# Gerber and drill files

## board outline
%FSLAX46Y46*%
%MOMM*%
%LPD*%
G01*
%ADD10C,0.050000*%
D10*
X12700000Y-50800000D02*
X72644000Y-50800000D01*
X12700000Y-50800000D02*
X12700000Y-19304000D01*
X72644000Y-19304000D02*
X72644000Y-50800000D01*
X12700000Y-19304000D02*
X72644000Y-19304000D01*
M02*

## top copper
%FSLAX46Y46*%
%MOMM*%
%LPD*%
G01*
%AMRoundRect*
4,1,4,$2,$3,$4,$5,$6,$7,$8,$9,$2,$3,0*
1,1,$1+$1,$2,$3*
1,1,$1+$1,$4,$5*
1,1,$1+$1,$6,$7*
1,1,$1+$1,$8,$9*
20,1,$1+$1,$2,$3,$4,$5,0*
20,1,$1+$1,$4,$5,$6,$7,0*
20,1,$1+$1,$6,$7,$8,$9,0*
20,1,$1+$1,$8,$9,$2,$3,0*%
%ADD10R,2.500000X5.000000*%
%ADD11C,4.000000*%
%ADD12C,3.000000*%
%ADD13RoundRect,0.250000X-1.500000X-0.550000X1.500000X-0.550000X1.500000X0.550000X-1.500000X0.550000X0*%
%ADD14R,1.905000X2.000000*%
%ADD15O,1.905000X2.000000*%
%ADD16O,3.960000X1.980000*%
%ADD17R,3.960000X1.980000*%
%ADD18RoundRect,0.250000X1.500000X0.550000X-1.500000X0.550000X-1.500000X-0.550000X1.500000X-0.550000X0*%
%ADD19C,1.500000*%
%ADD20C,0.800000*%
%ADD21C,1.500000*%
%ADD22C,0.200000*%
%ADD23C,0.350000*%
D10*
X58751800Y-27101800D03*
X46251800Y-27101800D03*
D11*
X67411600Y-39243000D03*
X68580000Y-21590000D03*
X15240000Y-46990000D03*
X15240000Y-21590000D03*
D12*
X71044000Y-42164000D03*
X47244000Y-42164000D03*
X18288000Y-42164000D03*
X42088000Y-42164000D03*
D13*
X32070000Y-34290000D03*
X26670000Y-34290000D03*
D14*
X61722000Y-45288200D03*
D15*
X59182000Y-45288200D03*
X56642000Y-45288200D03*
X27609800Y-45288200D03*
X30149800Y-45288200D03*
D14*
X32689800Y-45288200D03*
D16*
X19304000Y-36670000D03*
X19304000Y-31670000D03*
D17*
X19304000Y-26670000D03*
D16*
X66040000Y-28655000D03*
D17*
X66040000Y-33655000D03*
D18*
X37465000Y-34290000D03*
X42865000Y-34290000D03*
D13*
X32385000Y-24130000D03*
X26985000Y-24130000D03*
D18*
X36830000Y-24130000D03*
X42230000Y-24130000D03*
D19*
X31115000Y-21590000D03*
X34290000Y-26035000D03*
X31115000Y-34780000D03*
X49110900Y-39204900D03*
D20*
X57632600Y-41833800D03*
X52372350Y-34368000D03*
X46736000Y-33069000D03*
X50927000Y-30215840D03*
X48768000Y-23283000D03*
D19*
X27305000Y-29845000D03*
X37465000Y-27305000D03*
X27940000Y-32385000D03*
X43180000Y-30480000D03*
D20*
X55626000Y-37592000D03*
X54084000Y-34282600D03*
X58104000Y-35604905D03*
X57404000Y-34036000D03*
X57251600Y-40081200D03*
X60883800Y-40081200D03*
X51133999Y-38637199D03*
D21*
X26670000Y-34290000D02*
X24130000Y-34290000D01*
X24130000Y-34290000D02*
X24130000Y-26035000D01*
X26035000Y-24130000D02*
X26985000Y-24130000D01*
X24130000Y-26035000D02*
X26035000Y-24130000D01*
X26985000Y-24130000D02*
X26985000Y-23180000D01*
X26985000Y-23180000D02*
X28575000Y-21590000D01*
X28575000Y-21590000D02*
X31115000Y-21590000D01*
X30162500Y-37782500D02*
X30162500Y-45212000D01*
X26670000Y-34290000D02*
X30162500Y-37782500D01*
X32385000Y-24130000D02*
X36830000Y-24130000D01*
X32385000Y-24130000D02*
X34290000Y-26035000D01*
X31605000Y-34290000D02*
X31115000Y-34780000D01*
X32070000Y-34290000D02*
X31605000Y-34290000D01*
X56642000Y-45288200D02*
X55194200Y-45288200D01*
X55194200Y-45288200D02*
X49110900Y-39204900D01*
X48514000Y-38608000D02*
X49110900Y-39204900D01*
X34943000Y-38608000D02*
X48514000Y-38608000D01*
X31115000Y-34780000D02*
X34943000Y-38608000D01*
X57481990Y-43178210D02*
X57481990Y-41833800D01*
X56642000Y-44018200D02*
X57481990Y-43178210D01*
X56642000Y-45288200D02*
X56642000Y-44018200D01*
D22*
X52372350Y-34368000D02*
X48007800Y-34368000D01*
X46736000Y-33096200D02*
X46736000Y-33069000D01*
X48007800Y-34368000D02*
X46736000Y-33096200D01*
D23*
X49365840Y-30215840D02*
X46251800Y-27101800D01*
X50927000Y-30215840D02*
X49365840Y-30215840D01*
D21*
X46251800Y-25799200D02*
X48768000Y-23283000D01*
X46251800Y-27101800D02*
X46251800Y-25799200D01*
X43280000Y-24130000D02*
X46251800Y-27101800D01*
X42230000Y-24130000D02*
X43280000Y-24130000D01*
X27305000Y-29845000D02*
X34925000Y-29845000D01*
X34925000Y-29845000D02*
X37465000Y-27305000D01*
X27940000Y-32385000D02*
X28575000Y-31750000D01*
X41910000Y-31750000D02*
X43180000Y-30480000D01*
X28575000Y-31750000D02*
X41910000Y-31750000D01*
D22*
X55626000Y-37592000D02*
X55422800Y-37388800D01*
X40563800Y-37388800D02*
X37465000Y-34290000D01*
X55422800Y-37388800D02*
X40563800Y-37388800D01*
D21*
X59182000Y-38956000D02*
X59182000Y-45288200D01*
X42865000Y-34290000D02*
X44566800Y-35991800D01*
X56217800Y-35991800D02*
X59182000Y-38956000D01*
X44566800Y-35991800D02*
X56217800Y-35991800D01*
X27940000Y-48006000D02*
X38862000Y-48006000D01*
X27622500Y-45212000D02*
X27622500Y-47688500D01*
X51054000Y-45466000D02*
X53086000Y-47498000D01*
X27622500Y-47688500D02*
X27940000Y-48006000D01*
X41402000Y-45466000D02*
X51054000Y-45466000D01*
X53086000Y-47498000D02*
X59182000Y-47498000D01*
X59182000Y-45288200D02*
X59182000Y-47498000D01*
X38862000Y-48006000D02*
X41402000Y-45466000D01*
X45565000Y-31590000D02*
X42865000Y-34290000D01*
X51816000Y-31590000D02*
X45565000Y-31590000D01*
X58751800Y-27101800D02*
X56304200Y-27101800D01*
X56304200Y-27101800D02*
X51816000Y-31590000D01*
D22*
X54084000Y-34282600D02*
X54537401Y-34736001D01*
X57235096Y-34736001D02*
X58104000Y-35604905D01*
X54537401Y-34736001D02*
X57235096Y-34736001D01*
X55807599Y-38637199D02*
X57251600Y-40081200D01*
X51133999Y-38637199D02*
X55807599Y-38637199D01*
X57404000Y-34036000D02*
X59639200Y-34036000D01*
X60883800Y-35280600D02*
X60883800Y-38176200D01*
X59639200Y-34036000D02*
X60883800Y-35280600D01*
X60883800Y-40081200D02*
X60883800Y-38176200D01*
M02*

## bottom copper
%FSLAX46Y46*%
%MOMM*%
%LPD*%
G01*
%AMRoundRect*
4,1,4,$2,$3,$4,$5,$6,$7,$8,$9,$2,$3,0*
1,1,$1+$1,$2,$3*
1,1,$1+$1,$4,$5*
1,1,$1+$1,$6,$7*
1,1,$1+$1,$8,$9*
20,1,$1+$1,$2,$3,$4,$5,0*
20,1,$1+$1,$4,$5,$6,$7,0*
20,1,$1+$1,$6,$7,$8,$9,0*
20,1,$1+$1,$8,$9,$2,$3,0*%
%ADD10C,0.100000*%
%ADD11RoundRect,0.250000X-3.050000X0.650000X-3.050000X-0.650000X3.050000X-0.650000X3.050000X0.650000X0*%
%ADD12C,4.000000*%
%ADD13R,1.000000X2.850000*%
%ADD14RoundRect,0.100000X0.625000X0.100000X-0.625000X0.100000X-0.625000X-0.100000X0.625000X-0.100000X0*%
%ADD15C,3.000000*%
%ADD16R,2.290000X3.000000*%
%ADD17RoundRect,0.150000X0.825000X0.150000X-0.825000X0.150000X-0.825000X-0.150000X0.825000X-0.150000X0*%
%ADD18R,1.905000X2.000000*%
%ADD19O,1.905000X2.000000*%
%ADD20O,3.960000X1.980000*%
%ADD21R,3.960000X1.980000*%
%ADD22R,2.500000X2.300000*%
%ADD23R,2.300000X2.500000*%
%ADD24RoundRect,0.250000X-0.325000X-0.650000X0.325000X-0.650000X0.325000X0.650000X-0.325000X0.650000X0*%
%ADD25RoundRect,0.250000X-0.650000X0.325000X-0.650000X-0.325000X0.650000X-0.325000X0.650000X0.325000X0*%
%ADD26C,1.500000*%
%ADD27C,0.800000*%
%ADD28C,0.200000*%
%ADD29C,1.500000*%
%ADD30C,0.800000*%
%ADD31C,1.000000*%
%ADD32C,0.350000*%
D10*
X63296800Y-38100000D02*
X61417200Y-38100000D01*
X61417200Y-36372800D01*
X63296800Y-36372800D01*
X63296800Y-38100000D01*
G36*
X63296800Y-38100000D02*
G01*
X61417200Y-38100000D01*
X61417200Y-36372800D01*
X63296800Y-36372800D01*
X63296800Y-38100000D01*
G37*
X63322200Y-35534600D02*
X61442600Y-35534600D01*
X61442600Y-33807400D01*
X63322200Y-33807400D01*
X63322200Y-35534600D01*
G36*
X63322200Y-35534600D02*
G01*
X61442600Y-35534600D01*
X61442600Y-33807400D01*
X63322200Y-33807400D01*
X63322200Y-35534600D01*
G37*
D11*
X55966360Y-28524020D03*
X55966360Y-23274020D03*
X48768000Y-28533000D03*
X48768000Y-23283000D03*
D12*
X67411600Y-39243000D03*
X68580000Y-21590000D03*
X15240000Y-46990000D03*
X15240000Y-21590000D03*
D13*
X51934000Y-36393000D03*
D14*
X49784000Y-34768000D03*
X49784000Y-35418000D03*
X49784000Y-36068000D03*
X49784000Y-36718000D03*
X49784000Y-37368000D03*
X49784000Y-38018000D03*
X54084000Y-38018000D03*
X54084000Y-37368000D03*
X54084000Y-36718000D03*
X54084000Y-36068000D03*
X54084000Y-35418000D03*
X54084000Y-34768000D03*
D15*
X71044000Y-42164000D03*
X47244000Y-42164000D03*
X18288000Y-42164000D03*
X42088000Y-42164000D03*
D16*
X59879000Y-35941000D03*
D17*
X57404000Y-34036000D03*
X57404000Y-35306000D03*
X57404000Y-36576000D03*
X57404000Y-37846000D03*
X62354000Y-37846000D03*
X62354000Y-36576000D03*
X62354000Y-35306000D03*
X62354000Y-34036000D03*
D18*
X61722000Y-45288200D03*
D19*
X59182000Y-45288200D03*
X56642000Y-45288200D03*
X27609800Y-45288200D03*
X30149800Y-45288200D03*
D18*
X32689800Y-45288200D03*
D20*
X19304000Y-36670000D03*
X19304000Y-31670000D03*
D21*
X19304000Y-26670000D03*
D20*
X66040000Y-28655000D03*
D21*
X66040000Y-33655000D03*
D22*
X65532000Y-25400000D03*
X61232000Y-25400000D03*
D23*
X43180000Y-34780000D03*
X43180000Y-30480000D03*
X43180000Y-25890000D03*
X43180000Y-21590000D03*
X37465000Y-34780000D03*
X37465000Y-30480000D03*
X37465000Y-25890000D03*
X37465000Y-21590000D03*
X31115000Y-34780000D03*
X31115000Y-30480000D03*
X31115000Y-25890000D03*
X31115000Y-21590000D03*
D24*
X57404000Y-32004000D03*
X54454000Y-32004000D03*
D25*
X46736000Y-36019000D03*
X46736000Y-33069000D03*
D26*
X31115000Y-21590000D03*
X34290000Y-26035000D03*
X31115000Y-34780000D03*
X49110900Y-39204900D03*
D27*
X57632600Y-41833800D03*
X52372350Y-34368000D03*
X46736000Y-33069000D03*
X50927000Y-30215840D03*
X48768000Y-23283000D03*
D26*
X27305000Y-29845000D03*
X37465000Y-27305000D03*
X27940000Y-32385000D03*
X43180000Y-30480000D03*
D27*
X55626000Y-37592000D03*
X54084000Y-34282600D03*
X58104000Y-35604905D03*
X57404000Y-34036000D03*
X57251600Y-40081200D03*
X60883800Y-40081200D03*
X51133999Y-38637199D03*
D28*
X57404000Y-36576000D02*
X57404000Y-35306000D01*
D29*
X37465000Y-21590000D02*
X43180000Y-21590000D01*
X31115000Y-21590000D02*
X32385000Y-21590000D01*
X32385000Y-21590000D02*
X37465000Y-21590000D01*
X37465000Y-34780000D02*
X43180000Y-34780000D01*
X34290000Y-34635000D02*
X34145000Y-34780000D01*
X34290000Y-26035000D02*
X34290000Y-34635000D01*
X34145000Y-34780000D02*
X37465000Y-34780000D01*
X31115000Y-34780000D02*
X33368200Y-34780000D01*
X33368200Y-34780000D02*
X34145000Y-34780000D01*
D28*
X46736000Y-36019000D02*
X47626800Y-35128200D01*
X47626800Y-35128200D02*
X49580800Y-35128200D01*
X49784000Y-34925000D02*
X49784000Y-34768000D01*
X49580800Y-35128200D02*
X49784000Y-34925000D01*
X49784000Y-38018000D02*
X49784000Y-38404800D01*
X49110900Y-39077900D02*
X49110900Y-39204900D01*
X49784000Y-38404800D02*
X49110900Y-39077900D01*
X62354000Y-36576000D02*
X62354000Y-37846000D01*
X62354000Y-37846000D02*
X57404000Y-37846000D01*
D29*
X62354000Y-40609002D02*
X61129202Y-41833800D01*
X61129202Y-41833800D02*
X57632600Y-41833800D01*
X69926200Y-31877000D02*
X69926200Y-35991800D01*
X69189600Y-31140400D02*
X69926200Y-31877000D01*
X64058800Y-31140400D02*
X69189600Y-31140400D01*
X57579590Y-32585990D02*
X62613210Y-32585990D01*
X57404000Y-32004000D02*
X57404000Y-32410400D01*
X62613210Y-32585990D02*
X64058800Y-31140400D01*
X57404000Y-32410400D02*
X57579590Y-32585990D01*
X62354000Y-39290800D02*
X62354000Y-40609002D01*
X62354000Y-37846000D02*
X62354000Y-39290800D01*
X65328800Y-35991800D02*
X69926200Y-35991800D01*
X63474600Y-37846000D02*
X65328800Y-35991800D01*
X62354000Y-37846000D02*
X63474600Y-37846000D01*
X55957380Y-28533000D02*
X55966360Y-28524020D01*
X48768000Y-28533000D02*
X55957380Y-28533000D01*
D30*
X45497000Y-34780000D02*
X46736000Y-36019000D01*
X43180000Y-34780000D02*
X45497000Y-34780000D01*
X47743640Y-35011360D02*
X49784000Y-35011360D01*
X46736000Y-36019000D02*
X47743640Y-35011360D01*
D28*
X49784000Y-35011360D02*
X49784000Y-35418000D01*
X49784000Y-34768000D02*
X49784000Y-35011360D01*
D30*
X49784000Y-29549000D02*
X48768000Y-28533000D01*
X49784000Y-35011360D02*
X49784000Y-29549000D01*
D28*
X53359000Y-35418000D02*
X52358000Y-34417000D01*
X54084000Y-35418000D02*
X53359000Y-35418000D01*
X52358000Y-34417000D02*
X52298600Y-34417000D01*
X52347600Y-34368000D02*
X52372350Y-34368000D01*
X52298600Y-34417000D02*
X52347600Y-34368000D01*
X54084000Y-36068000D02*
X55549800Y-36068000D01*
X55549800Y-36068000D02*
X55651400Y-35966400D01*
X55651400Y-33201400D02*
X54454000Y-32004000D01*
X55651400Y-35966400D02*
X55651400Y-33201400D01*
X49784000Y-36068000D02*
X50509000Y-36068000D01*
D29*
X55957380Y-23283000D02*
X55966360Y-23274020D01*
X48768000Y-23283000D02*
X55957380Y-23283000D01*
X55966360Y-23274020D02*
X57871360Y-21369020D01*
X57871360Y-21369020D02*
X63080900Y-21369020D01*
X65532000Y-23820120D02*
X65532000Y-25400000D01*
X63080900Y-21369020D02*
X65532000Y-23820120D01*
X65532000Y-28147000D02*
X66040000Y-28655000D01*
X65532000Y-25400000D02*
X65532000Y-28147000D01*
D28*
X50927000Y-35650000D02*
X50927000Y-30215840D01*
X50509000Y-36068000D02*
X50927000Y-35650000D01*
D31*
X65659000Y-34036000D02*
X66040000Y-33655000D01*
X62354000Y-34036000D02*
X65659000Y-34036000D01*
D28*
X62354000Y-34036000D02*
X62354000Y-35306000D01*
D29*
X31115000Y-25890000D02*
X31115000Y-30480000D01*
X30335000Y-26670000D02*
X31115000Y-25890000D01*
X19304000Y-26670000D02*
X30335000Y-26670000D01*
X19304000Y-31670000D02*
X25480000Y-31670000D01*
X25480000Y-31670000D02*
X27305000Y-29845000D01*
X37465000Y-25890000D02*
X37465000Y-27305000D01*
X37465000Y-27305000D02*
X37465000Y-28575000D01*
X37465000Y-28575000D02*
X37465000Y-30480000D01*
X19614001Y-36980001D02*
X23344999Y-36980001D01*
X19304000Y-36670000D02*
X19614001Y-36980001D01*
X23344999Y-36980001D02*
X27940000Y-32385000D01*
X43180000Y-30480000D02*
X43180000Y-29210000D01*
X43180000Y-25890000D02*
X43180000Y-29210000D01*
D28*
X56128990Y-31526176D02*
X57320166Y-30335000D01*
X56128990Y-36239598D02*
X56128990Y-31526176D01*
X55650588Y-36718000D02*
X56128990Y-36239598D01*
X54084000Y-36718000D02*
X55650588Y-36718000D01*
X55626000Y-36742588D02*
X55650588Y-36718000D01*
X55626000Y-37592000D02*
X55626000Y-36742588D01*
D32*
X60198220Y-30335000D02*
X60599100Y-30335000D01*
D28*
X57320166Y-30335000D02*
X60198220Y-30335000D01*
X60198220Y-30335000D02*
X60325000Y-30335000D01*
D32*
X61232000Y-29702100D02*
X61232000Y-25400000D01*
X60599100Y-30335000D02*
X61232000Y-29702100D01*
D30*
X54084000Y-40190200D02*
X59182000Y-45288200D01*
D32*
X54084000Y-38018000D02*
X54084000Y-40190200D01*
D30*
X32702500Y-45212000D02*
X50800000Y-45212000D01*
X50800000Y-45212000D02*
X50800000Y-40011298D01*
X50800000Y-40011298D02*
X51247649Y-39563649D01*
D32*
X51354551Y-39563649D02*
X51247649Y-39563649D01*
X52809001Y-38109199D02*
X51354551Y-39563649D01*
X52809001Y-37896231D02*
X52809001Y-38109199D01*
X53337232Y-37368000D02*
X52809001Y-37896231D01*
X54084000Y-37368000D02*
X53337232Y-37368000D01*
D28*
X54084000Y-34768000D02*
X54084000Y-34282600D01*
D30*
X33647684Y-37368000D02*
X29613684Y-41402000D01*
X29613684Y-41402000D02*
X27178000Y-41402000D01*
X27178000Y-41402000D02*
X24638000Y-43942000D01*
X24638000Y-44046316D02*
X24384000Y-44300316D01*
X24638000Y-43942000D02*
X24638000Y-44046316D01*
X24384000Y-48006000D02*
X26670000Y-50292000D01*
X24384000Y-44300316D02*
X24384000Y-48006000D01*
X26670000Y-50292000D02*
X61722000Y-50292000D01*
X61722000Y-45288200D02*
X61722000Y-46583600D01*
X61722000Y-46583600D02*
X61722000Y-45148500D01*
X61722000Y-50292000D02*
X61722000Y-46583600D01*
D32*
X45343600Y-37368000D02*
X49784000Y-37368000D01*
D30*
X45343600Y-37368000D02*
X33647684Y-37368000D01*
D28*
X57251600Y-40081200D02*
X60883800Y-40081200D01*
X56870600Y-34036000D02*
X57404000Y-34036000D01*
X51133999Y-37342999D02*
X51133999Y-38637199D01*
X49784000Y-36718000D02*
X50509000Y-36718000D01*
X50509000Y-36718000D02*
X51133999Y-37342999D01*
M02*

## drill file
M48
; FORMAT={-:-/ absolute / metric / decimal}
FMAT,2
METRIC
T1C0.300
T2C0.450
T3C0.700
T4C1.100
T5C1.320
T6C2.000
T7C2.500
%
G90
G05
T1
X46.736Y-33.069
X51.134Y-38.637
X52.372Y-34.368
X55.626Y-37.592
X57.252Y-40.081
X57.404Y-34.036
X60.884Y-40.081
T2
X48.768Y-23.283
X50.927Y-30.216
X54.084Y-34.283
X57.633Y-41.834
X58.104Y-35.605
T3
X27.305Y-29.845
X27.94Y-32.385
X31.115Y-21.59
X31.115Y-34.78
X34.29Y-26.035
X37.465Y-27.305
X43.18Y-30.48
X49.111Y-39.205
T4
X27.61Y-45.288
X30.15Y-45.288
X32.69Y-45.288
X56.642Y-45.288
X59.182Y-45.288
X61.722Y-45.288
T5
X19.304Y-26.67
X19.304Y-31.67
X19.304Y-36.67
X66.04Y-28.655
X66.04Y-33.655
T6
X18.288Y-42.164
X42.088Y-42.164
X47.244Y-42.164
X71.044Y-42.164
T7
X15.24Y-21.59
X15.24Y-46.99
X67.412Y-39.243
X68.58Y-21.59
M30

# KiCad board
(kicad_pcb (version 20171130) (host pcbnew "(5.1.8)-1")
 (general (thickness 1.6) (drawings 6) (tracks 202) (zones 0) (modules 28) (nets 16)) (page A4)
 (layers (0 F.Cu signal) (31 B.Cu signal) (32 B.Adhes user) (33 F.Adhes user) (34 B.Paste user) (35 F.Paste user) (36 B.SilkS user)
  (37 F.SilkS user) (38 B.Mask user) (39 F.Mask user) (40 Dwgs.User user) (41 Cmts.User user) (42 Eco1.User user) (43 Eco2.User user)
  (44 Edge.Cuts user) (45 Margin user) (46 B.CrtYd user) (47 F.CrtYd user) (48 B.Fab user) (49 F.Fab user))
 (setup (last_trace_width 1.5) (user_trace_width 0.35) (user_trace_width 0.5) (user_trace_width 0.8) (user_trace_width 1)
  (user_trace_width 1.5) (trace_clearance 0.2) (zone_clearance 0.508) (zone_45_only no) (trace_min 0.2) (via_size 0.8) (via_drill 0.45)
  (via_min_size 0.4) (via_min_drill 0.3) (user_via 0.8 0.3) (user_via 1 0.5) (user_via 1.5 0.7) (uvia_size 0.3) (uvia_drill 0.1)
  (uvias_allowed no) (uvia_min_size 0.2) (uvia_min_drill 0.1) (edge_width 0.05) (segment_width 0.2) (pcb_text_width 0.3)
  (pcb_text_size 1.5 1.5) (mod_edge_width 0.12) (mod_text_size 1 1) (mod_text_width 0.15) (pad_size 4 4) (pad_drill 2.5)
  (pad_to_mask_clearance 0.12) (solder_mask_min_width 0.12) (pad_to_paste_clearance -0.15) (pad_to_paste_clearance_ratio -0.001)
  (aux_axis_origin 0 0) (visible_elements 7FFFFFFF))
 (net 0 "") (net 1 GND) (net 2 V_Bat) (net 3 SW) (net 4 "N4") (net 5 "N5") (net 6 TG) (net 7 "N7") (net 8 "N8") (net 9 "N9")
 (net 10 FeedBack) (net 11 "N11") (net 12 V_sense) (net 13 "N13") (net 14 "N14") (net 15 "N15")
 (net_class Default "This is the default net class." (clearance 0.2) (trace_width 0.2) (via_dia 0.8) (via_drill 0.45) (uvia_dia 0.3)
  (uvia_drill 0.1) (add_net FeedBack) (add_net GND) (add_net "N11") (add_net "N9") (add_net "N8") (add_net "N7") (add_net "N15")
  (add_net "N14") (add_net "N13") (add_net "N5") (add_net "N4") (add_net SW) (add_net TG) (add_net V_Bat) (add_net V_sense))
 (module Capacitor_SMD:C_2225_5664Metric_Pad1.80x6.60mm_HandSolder (layer B.Cu) (at 55.96636 25.89902 270)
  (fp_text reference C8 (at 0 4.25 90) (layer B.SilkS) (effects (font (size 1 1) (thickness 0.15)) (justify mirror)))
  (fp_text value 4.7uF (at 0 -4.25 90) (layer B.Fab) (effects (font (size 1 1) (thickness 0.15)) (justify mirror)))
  (pad 2 smd roundrect (at 2.625 0 270) (size 1.8 6.6) (layers B.Cu B.Paste B.Mask) (roundrect_rratio 0.138889) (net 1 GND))
  (pad 1 smd roundrect (at -2.625 0 270) (size 1.8 6.6) (layers B.Cu B.Paste B.Mask) (roundrect_rratio 0.138889) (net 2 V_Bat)))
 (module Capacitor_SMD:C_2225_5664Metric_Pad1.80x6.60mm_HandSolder (layer B.Cu) (at 48.768 25.908 270)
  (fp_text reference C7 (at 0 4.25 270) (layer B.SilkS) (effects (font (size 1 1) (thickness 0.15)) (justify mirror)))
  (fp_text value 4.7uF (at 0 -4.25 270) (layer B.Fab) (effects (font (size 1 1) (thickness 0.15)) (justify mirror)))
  (pad 2 smd roundrect (at 2.625 0 270) (size 1.8 6.6) (layers B.Cu B.Paste B.Mask) (roundrect_rratio 0.138889) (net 1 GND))
  (pad 1 smd roundrect (at -2.625 0 270) (size 1.8 6.6) (layers B.Cu B.Paste B.Mask) (roundrect_rratio 0.138889) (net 2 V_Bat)))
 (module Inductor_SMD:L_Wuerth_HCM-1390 (layer F.Cu) (at 52.5018 27.1018)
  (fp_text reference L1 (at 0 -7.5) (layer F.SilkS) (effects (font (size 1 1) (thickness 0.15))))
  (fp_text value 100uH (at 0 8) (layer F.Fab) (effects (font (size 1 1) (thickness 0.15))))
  (pad 2 smd rect (at 6.25 0) (size 2.5 5) (layers F.Cu F.Paste F.Mask) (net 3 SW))
  (pad 1 smd rect (at -6.25 0) (size 2.5 5) (layers F.Cu F.Paste F.Mask) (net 2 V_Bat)))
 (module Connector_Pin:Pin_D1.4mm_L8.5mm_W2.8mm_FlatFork (layer F.Cu) (at 67.4116 39.243)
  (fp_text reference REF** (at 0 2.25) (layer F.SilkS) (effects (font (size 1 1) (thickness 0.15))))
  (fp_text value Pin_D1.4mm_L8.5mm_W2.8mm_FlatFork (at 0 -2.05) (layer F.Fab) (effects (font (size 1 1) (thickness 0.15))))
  (pad 1 thru_hole circle (at 0 0) (size 4 4) (drill 2.5) (layers *.Cu *.Mask)))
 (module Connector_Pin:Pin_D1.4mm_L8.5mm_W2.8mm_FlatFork (layer F.Cu) (at 68.58 21.59)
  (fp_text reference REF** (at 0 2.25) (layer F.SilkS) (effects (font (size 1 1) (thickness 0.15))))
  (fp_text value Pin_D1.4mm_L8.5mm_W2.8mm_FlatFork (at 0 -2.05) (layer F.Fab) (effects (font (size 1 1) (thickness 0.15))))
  (pad 1 thru_hole circle (at 0 0) (size 4 4) (drill 2.5) (layers *.Cu *.Mask)))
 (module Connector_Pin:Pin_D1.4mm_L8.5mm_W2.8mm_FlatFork (layer F.Cu) (at 15.24 46.99)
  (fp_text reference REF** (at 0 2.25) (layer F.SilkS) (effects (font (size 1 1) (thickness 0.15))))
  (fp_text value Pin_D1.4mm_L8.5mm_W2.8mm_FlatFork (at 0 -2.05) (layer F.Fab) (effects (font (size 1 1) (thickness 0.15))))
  (pad 1 thru_hole circle (at 0 0) (size 4 4) (drill 2.5) (layers *.Cu *.Mask)))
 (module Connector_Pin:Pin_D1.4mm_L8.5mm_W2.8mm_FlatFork (layer F.Cu) (at 15.24 21.59)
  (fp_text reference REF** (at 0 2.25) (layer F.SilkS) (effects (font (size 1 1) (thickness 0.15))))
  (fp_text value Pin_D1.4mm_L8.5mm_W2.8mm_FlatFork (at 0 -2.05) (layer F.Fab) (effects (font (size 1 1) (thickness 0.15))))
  (pad 1 thru_hole circle (at 0 0) (size 4 4) (drill 2.5) (layers *.Cu *.Mask)))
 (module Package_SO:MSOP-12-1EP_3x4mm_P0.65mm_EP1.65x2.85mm (layer B.Cu) (at 51.934 36.393 180)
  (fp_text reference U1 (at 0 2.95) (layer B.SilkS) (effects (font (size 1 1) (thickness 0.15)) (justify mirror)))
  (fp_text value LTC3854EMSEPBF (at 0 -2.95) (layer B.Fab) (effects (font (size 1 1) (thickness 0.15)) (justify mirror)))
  (pad "" smd roundrect (at 0.41 -0.71 180) (size 0.67 1.15) (layers B.Paste) (roundrect_rratio 0.25))
  (pad "" smd roundrect (at 0.41 0.71 180) (size 0.67 1.15) (layers B.Paste) (roundrect_rratio 0.25))
  (pad "" smd roundrect (at -0.41 -0.71 180) (size 0.67 1.15) (layers B.Paste) (roundrect_rratio 0.25))
  (pad "" smd roundrect (at -0.41 0.71 180) (size 0.67 1.15) (layers B.Paste) (roundrect_rratio 0.25))
  (pad 13 smd rect (at 0 0 180) (size 1 2.85) (layers B.Cu B.Mask))
  (pad 12 smd roundrect (at 2.15 1.625 180) (size 1.45 0.4) (layers B.Cu B.Paste B.Mask) (roundrect_rratio 0.25) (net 1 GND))
  (pad 11 smd roundrect (at 2.15 0.975 180) (size 1.45 0.4) (layers B.Cu B.Paste B.Mask) (roundrect_rratio 0.25) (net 1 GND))
  (pad 10 smd roundrect (at 2.15 0.325 180) (size 1.45 0.4) (layers B.Cu B.Paste B.Mask) (roundrect_rratio 0.25) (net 2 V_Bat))
  (pad 9 smd roundrect (at 2.15 -0.325 180) (size 1.45 0.4) (layers B.Cu B.Paste B.Mask) (roundrect_rratio 0.25) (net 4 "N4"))
  (pad 8 smd roundrect (at 2.15 -0.975 180) (size 1.45 0.4) (layers B.Cu B.Paste B.Mask) (roundrect_rratio 0.25) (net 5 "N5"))
  (pad 7 smd roundrect (at 2.15 -1.625 180) (size 1.45 0.4) (layers B.Cu B.Paste B.Mask) (roundrect_rratio 0.25) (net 1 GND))
  (pad 6 smd roundrect (at -2.15 -1.625 180) (size 1.45 0.4) (layers B.Cu B.Paste B.Mask) (roundrect_rratio 0.25) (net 3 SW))
  (pad 5 smd roundrect (at -2.15 -0.975 180) (size 1.45 0.4) (layers B.Cu B.Paste B.Mask) (roundrect_rratio 0.25) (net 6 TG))
  (pad 4 smd roundrect (at -2.15 -0.325 180) (size 1.45 0.4) (layers B.Cu B.Paste B.Mask) (roundrect_rratio 0.25) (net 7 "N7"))
  (pad 3 smd roundrect (at -2.15 0.325 180) (size 1.45 0.4) (layers B.Cu B.Paste B.Mask) (roundrect_rratio 0.25) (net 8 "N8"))
  (pad 2 smd roundrect (at -2.15 0.975 180) (size 1.45 0.4) (layers B.Cu B.Paste B.Mask) (roundrect_rratio 0.25) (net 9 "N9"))
  (pad 1 smd roundrect (at -2.15 1.625 180) (size 1.45 0.4) (layers B.Cu B.Paste B.Mask) (roundrect_rratio 0.25) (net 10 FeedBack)))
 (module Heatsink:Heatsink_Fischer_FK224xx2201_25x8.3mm (layer F.Cu) (at 47.244 42.164)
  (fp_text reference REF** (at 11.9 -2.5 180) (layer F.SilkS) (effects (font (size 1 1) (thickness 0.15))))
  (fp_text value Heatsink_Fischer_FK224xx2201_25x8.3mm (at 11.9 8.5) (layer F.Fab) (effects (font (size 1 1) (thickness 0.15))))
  (pad 1 thru_hole circle (at 23.8 0) (size 3 3) (drill 2) (layers *.Cu *.Mask))
  (pad 1 thru_hole circle (at 0 0) (size 3 3) (drill 2) (layers *.Cu *.Mask)))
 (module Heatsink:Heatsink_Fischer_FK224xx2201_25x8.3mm (layer F.Cu) (at 18.288 42.164)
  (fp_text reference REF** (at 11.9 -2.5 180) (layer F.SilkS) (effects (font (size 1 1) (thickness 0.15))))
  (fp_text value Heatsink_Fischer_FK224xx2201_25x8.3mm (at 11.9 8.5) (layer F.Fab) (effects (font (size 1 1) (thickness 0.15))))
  (pad 1 thru_hole circle (at 0 0) (size 3 3) (drill 2) (layers *.Cu *.Mask))
  (pad 1 thru_hole circle (at 23.8 0) (size 3 3) (drill 2) (layers *.Cu *.Mask)))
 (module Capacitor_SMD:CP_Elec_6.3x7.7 (layer F.Cu) (at 29.37 34.29)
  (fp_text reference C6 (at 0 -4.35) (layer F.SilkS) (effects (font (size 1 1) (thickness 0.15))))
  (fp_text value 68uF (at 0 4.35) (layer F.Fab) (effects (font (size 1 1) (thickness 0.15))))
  (pad 2 smd roundrect (at 2.7 0) (size 3.5 1.6) (layers F.Cu F.Paste F.Mask) (roundrect_rratio 0.15625) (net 1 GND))
  (pad 1 smd roundrect (at -2.7 0) (size 3.5 1.6) (layers F.Cu F.Paste F.Mask) (roundrect_rratio 0.15625) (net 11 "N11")))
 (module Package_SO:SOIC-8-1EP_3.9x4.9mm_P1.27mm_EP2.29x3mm (layer B.Cu) (at 59.879 35.941 180)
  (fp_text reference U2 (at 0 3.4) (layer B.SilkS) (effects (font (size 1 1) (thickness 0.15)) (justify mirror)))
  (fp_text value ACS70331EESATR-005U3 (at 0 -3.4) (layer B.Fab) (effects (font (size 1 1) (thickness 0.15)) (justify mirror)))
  (pad "" smd roundrect (at 0.57 -0.75 180) (size 0.92 1.21) (layers B.Paste) (roundrect_rratio 0.25))
  (pad "" smd roundrect (at 0.57 0.75 180) (size 0.92 1.21) (layers B.Paste) (roundrect_rratio 0.25))
  (pad "" smd roundrect (at -0.57 -0.75 180) (size 0.92 1.21) (layers B.Paste) (roundrect_rratio 0.25))
  (pad "" smd roundrect (at -0.57 0.75 180) (size 0.92 1.21) (layers B.Paste) (roundrect_rratio 0.25))
  (pad 9 smd rect (at 0 0 180) (size 2.29 3) (layers B.Cu B.Mask))
  (pad 8 smd roundrect (at 2.475 1.905 180) (size 1.95 0.6) (layers B.Cu B.Paste B.Mask) (roundrect_rratio 0.25) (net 4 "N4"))
  (pad 7 smd roundrect (at 2.475 0.635 180) (size 1.95 0.6) (layers B.Cu B.Paste B.Mask) (roundrect_rratio 0.25) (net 10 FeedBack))
  (pad 6 smd roundrect (at 2.475 -0.635 180) (size 1.95 0.6) (layers B.Cu B.Paste B.Mask) (roundrect_rratio 0.25))
  (pad 5 smd roundrect (at 2.475 -1.905 180) (size 1.95 0.6) (layers B.Cu B.Paste B.Mask) (roundrect_rratio 0.25) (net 1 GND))
  (pad 4 smd roundrect (at -2.475 -1.905 180) (size 1.95 0.6) (layers B.Cu B.Paste B.Mask) (roundrect_rratio 0.25) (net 1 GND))
  (pad 3 smd roundrect (at -2.475 -0.635 180) (size 1.95 0.6) (layers B.Cu B.Paste B.Mask) (roundrect_rratio 0.25) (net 1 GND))
  (pad 2 smd roundrect (at -2.475 0.635 180) (size 1.95 0.6) (layers B.Cu B.Paste B.Mask) (roundrect_rratio 0.25) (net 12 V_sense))
  (pad 1 smd roundrect (at -2.475 1.905 180) (size 1.95 0.6) (layers B.Cu B.Paste B.Mask) (roundrect_rratio 0.25) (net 12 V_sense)))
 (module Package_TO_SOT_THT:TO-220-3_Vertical (layer F.Cu) (at 61.722 45.2882 180)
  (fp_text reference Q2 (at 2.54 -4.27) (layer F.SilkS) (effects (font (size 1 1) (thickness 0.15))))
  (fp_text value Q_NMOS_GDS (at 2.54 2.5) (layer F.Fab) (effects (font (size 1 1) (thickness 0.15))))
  (pad 1 thru_hole rect (at 0 0 180) (size 1.905 2) (drill 1.1) (layers *.Cu *.Mask) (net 5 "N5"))
  (pad 2 thru_hole oval (at 2.54 0 180) (size 1.905 2) (drill 1.1) (layers *.Cu *.Mask) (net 3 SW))
  (pad 3 thru_hole oval (at 5.08 0 180) (size 1.905 2) (drill 1.1) (layers *.Cu *.Mask) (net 1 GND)))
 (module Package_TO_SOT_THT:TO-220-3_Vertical (layer F.Cu) (at 32.6898 45.2882 180)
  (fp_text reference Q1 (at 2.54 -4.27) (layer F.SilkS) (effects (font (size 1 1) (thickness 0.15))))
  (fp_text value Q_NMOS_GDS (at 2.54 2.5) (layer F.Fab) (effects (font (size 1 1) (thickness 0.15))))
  (pad 3 thru_hole oval (at 5.08 0 180) (size 1.905 2) (drill 1.1) (layers *.Cu *.Mask) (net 3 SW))
  (pad 2 thru_hole oval (at 2.54 0 180) (size 1.905 2) (drill 1.1) (layers *.Cu *.Mask) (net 11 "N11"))
  (pad 1 thru_hole rect (at 0 0 180) (size 1.905 2) (drill 1.1) (layers *.Cu *.Mask) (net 6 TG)))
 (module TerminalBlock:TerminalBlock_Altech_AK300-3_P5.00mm (layer F.Cu) (at 19.304 26.67 270)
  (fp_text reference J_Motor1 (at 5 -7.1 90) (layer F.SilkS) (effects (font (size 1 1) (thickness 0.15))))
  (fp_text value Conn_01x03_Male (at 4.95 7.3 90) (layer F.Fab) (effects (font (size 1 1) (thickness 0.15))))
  (pad 3 thru_hole oval (at 10 0 270) (size 1.98 3.96) (drill 1.32) (layers *.Cu *.Mask) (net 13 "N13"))
  (pad 2 thru_hole oval (at 5 0 270) (size 1.98 3.96) (drill 1.32) (layers *.Cu *.Mask) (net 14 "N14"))
  (pad 1 thru_hole rect (at 0 0 270) (size 1.98 3.96) (drill 1.32) (layers *.Cu *.Mask) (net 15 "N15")))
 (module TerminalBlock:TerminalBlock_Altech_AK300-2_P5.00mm (layer F.Cu) (at 66.04 33.655 90)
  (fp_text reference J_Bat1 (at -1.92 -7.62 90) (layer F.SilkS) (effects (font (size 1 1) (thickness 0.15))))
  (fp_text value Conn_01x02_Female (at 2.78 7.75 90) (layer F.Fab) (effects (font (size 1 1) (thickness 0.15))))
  (pad 2 thru_hole oval (at 5 0 90) (size 1.98 3.96) (drill 1.32) (layers *.Cu *.Mask) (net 2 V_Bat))
  (pad 1 thru_hole rect (at 0 0 90) (size 1.98 3.96) (drill 1.32) (layers *.Cu *.Mask) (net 12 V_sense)))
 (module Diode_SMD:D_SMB (layer B.Cu) (at 63.382 25.4)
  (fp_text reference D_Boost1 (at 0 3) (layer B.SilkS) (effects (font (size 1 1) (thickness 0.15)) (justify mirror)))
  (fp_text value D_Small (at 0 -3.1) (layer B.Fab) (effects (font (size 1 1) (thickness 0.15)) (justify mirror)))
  (pad 2 smd rect (at 2.15 0) (size 2.5 2.3) (layers B.Cu B.Paste B.Mask) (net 2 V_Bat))
  (pad 1 smd rect (at -2.15 0) (size 2.5 2.3) (layers B.Cu B.Paste B.Mask) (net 7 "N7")))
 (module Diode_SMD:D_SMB (layer B.Cu) (at 43.18 32.63 270)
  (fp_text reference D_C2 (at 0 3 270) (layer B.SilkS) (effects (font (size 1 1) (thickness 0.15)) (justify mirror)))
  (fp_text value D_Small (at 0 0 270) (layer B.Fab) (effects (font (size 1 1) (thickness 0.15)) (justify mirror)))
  (pad 2 smd rect (at 2.15 0 270) (size 2.5 2.3) (layers B.Cu B.Paste B.Mask) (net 1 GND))
  (pad 1 smd rect (at -2.15 0 270) (size 2.5 2.3) (layers B.Cu B.Paste B.Mask) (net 13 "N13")))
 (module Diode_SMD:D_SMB (layer B.Cu) (at 43.18 23.74 270)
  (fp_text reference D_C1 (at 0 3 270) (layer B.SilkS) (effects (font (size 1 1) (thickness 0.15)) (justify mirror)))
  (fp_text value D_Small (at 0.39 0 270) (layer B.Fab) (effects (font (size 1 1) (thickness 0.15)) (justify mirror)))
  (pad 2 smd rect (at 2.15 0 270) (size 2.5 2.3) (layers B.Cu B.Paste B.Mask) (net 13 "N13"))
  (pad 1 smd rect (at -2.15 0 270) (size 2.5 2.3) (layers B.Cu B.Paste B.Mask) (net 11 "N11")))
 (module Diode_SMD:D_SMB (layer B.Cu) (at 37.465 32.63 270)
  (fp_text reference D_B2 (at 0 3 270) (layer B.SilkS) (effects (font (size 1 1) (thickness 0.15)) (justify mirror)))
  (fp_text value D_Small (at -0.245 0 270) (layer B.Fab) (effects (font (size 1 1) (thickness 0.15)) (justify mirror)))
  (pad 2 smd rect (at 2.15 0 270) (size 2.5 2.3) (layers B.Cu B.Paste B.Mask) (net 1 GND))
  (pad 1 smd rect (at -2.15 0 270) (size 2.5 2.3) (layers B.Cu B.Paste B.Mask) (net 14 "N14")))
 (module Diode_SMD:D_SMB (layer B.Cu) (at 37.465 23.74 270)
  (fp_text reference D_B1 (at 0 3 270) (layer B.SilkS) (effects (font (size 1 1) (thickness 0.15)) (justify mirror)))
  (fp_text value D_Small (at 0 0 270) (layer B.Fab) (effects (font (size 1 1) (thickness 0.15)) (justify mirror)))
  (pad 2 smd rect (at 2.15 0 270) (size 2.5 2.3) (layers B.Cu B.Paste B.Mask) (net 14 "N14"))
  (pad 1 smd rect (at -2.15 0 270) (size 2.5 2.3) (layers B.Cu B.Paste B.Mask) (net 11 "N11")))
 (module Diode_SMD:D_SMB (layer B.Cu) (at 31.115 32.63 270)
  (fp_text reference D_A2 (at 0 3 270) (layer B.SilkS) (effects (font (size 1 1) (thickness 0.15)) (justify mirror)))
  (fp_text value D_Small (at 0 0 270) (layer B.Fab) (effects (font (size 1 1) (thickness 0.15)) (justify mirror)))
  (pad 2 smd rect (at 2.15 0 270) (size 2.5 2.3) (layers B.Cu B.Paste B.Mask) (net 1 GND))
  (pad 1 smd rect (at -2.15 0 270) (size 2.5 2.3) (layers B.Cu B.Paste B.Mask) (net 15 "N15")))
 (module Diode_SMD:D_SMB (layer B.Cu) (at 31.115 23.74 270)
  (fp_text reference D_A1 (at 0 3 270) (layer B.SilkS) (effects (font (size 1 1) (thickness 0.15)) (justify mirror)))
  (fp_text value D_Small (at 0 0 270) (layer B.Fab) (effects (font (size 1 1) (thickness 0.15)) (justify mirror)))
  (pad 2 smd rect (at 2.15 0 270) (size 2.5 2.3) (layers B.Cu B.Paste B.Mask) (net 15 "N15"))
  (pad 1 smd rect (at -2.15 0 270) (size 2.5 2.3) (layers B.Cu B.Paste B.Mask) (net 11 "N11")))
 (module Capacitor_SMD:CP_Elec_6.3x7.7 (layer F.Cu) (at 40.165 34.29 180)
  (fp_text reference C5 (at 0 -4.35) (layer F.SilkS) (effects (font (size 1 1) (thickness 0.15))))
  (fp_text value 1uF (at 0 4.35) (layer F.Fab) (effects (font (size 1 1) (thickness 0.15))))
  (pad 2 smd roundrect (at 2.7 0 180) (size 3.5 1.6) (layers F.Cu F.Paste F.Mask) (roundrect_rratio 0.15625) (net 7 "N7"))
  (pad 1 smd roundrect (at -2.7 0 180) (size 3.5 1.6) (layers F.Cu F.Paste F.Mask) (roundrect_rratio 0.15625) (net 3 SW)))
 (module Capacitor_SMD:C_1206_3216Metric (layer B.Cu) (at 55.929 32.004)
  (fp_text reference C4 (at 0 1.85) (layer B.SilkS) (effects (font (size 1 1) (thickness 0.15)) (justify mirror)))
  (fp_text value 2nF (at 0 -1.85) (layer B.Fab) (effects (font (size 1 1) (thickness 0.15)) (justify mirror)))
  (pad 2 smd roundrect (at 1.475 0) (size 1.15 1.8) (layers B.Cu B.Paste B.Mask) (roundrect_rratio 0.217391) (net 1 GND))
  (pad 1 smd roundrect (at -1.475 0) (size 1.15 1.8) (layers B.Cu B.Paste B.Mask) (roundrect_rratio 0.217391) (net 8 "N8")))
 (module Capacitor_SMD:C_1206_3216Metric (layer B.Cu) (at 46.736 34.544 270)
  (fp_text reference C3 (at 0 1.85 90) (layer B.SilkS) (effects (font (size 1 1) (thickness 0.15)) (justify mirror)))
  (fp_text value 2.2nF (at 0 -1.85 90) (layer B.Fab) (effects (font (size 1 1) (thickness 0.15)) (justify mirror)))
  (pad 2 smd roundrect (at 1.475 0 270) (size 1.15 1.8) (layers B.Cu B.Paste B.Mask) (roundrect_rratio 0.217391) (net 1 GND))
  (pad 1 smd roundrect (at -1.475 0 270) (size 1.15 1.8) (layers B.Cu B.Paste B.Mask) (roundrect_rratio 0.217391) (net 9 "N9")))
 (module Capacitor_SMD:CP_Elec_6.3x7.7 (layer F.Cu) (at 29.685 24.13)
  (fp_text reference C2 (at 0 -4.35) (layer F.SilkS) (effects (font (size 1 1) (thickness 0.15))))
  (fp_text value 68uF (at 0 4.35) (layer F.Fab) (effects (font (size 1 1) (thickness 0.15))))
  (pad 2 smd roundrect (at 2.7 0) (size 3.5 1.6) (layers F.Cu F.Paste F.Mask) (roundrect_rratio 0.15625) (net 1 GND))
  (pad 1 smd roundrect (at -2.7 0) (size 3.5 1.6) (layers F.Cu F.Paste F.Mask) (roundrect_rratio 0.15625) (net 11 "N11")))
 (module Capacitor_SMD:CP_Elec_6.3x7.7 (layer F.Cu) (at 39.53 24.13 180)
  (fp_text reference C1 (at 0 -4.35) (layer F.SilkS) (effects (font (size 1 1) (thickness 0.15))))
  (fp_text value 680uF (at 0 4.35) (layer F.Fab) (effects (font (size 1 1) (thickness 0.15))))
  (pad 2 smd roundrect (at 2.7 0 180) (size 3.5 1.6) (layers F.Cu F.Paste F.Mask) (roundrect_rratio 0.15625) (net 1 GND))
  (pad 1 smd roundrect (at -2.7 0 180) (size 3.5 1.6) (layers F.Cu F.Paste F.Mask) (roundrect_rratio 0.15625) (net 2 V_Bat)))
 (gr_poly (pts (xy 63.2968 38.1) (xy 61.4172 38.1) (xy 61.4172 36.3728) (xy 63.2968 36.3728)) (layer B.Cu) (width 0.1))
 (gr_poly (pts (xy 63.3222 35.5346) (xy 61.4426 35.5346) (xy 61.4426 33.8074) (xy 63.3222 33.8074)) (layer B.Cu) (width 0.1))
 (gr_line (start 12.7 50.8) (end 72.644 50.8) (layer Edge.Cuts) (width 0.05))
 (gr_line (start 12.7 50.8) (end 12.7 19.304) (layer Edge.Cuts) (width 0.05))
 (gr_line (start 72.644 19.304) (end 72.644 50.8) (layer Edge.Cuts) (width 0.05))
 (gr_line (start 12.7 19.304) (end 72.644 19.304) (layer Edge.Cuts) (width 0.05))
 (segment (start 57.404 36.576) (end 57.404 35.306) (width 0.2) (layer B.Cu) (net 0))
 (segment (start 37.465 21.59) (end 43.18 21.59) (width 1.5) (layer B.Cu) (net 11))
 (segment (start 26.67 34.29) (end 24.13 34.29) (width 1.5) (layer F.Cu) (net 11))
 (segment (start 24.13 34.29) (end 24.13 26.035) (width 1.5) (layer F.Cu) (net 11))
 (segment (start 26.035 24.13) (end 26.985 24.13) (width 1.5) (layer F.Cu) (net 11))
 (segment (start 24.13 26.035) (end 26.035 24.13) (width 1.5) (layer F.Cu) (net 11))
 (segment (start 26.985 24.13) (end 26.985 23.18) (width 1.5) (layer F.Cu) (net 11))
 (segment (start 26.985 23.18) (end 28.575 21.59) (width 1.5) (layer F.Cu) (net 11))
 (via (at 31.115 21.59) (size 1.5) (drill 0.7) (layers F.Cu B.Cu) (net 11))
 (segment (start 28.575 21.59) (end 31.115 21.59) (width 1.5) (layer F.Cu) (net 11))
 (segment (start 31.115 21.59) (end 32.385 21.59) (width 1.5) (layer B.Cu) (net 11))
 (segment (start 32.385 21.59) (end 37.465 21.59) (width 1.5) (layer B.Cu) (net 11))
 (segment (start 30.1625 37.7825) (end 30.1625 45.212) (width 1.5) (layer F.Cu) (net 11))
 (segment (start 26.67 34.29) (end 30.1625 37.7825) (width 1.5) (layer F.Cu) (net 11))
 (segment (start 37.465 34.78) (end 43.18 34.78) (width 1.5) (layer B.Cu) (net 1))
 (segment (start 32.385 24.13) (end 36.83 24.13) (width 1.5) (layer F.Cu) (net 1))
 (segment (start 32.385 24.13) (end 34.29 26.035) (width 1.5) (layer F.Cu) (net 1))
 (via (at 34.29 26.035) (size 1.5) (drill 0.7) (layers F.Cu B.Cu) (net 1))
 (segment (start 34.29 34.635) (end 34.145 34.78) (width 1.5) (layer B.Cu) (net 1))
 (segment (start 34.29 26.035) (end 34.29 34.635) (width 1.5) (layer B.Cu) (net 1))
 (segment (start 34.145 34.78) (end 37.465 34.78) (width 1.5) (layer B.Cu) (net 1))
 (via (at 31.115 34.78) (size 1.5) (drill 0.7) (layers F.Cu B.Cu) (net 1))
 (segment (start 31.605 34.29) (end 31.115 34.78) (width 1.5) (layer F.Cu) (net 1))
 (segment (start 32.07 34.29) (end 31.605 34.29) (width 1.5) (layer F.Cu) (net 1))
 (segment (start 56.642 45.2882) (end 55.1942 45.2882) (width 1.5) (layer F.Cu) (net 1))
 (segment (start 31.115 34.78) (end 33.3682 34.78) (width 1.5) (layer B.Cu) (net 1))
 (segment (start 33.3682 34.78) (end 34.145 34.78) (width 1.5) (layer B.Cu) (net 1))
 (segment (start 46.736 36.019) (end 47.6268 35.1282) (width 0.2) (layer B.Cu) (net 1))
 (segment (start 47.6268 35.1282) (end 49.5808 35.1282) (width 0.2) (layer B.Cu) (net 1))
 (segment (start 49.784 34.925) (end 49.784 34.768) (width 0.2) (layer B.Cu) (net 1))
 (segment (start 49.5808 35.1282) (end 49.784 34.925) (width 0.2) (layer B.Cu) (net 1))
 (segment (start 49.784 38.018) (end 49.784 38.4048) (width 0.2) (layer B.Cu) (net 1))
 (segment (start 49.1109 39.0779) (end 49.1109 39.2049) (width 0.2) (layer B.Cu) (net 1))
 (segment (start 49.784 38.4048) (end 49.1109 39.0779) (width 0.2) (layer B.Cu) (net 1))
 (via (at 49.1109 39.2049) (size 1.5) (drill 0.7) (layers F.Cu B.Cu) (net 1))
 (segment (start 55.1942 45.2882) (end 49.1109 39.2049) (width 1.5) (layer F.Cu) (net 1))
 (segment (start 48.514 38.608) (end 49.1109 39.2049) (width 1.5) (layer F.Cu) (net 1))
 (segment (start 34.943 38.608) (end 48.514 38.608) (width 1.5) (layer F.Cu) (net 1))
 (segment (start 31.115 34.78) (end 34.943 38.608) (width 1.5) (layer F.Cu) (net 1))
 (segment (start 62.354 36.576) (end 62.354 37.846) (width 0.2) (layer B.Cu) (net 1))
 (segment (start 62.354 37.846) (end 57.404 37.846) (width 0.2) (layer B.Cu) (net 1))
 (segment (start 62.354 40.609002) (end 61.129202 41.8338) (width 1.5) (layer B.Cu) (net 1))
 (via (at 57.6326 41.8338) (size 0.8) (drill 0.45) (layers F.Cu B.Cu) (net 1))
 (segment (start 61.129202 41.8338) (end 57.6326 41.8338) (width 1.5) (layer B.Cu) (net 1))
 (segment (start 57.48199 43.17821) (end 57.48199 41.8338) (width 1.5) (layer F.Cu) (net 1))
 (segment (start 56.642 44.0182) (end 57.48199 43.17821) (width 1.5) (layer F.Cu) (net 1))
 (segment (start 56.642 45.2882) (end 56.642 44.0182) (width 1.5) (layer F.Cu) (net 1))
 (segment (start 69.9262 31.877) (end 69.9262 35.9918) (width 1.5) (layer B.Cu) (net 1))
 (segment (start 69.1896 31.1404) (end 69.9262 31.877) (width 1.5) (layer B.Cu) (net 1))
 (segment (start 64.0588 31.1404) (end 69.1896 31.1404) (width 1.5) (layer B.Cu) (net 1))
 (segment (start 57.57959 32.58599) (end 62.61321 32.58599) (width 1.5) (layer B.Cu) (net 1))
 (segment (start 57.404 32.004) (end 57.404 32.4104) (width 1.5) (layer B.Cu) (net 1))
 (segment (start 62.61321 32.58599) (end 64.0588 31.1404) (width 1.5) (layer B.Cu) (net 1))
 (segment (start 57.404 32.4104) (end 57.57959 32.58599) (width 1.5) (layer B.Cu) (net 1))
 (segment (start 62.354 39.2908) (end 62.354 40.609002) (width 1.5) (layer B.Cu) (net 1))
 (segment (start 62.354 37.846) (end 62.354 39.2908) (width 1.5) (layer B.Cu) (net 1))
 (segment (start 65.3288 35.9918) (end 69.9262 35.9918) (width 1.5) (layer B.Cu) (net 1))
 (segment (start 63.4746 37.846) (end 65.3288 35.9918) (width 1.5) (layer B.Cu) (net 1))
 (segment (start 62.354 37.846) (end 63.4746 37.846) (width 1.5) (layer B.Cu) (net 1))
 (segment (start 55.95738 28.533) (end 55.96636 28.52402) (width 1.5) (layer B.Cu) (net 1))
 (segment (start 48.768 28.533) (end 55.95738 28.533) (width 1.5) (layer B.Cu) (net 1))
 (segment (start 45.497 34.78) (end 46.736 36.019) (width 0.8) (layer B.Cu) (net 1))
 (segment (start 43.18 34.78) (end 45.497 34.78) (width 0.8) (layer B.Cu) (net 1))
 (segment (start 47.74364 35.01136) (end 49.784 35.01136) (width 0.8) (layer B.Cu) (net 1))
 (segment (start 46.736 36.019) (end 47.74364 35.01136) (width 0.8) (layer B.Cu) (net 1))
 (segment (start 49.784 35.01136) (end 49.784 35.418) (width 0.2) (layer B.Cu) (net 1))
 (segment (start 49.784 34.768) (end 49.784 35.01136) (width 0.2) (layer B.Cu) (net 1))
 (segment (start 49.784 29.549) (end 48.768 28.533) (width 0.8) (layer B.Cu) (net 1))
 (segment (start 49.784 35.01136) (end 49.784 29.549) (width 0.8) (layer B.Cu) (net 1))
 (segment (start 53.359 35.418) (end 52.358 34.417) (width 0.2) (layer B.Cu) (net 9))
 (segment (start 54.084 35.418) (end 53.359 35.418) (width 0.2) (layer B.Cu) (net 9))
 (segment (start 52.358 34.417) (end 52.2986 34.417) (width 0.2) (layer B.Cu) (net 9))
 (via (at 52.37235 34.368) (size 0.8) (drill 0.3) (layers F.Cu B.Cu) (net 9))
 (segment (start 52.3476 34.368) (end 52.37235 34.368) (width 0.2) (layer B.Cu) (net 9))
 (segment (start 52.2986 34.417) (end 52.3476 34.368) (width 0.2) (layer B.Cu) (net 9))
 (segment (start 52.37235 34.368) (end 48.0078 34.368) (width 0.2) (layer F.Cu) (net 9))
 (via (at 46.736 33.069) (size 0.8) (drill 0.3) (layers F.Cu B.Cu) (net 9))
 (segment (start 46.736 33.0962) (end 46.736 33.069) (width 0.2) (layer F.Cu) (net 9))
 (segment (start 48.0078 34.368) (end 46.736 33.0962) (width 0.2) (layer F.Cu) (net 9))
 (segment (start 54.084 36.068) (end 55.5498 36.068) (width 0.2) (layer B.Cu) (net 8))
 (segment (start 55.5498 36.068) (end 55.6514 35.9664) (width 0.2) (layer B.Cu) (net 8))
 (segment (start 55.6514 33.2014) (end 54.454 32.004) (width 0.2) (layer B.Cu) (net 8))
 (segment (start 55.6514 35.9664) (end 55.6514 33.2014) (width 0.2) (layer B.Cu) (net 8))
 (segment (start 49.784 36.068) (end 50.509 36.068) (width 0.2) (layer B.Cu) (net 2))
 (segment (start 55.95738 23.283) (end 55.96636 23.27402) (width 1.5) (layer B.Cu) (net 2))
 (segment (start 48.768 23.283) (end 55.95738 23.283) (width 1.5) (layer B.Cu) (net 2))
 (segment (start 55.96636 23.27402) (end 57.87136 21.36902) (width 1.5) (layer B.Cu) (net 2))
 (segment (start 57.87136 21.36902) (end 63.0809 21.36902) (width 1.5) (layer B.Cu) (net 2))
 (segment (start 65.532 23.82012) (end 65.532 25.4) (width 1.5) (layer B.Cu) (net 2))
 (segment (start 63.0809 21.36902) (end 65.532 23.82012) (width 1.5) (layer B.Cu) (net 2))
 (segment (start 65.532 28.147) (end 66.04 28.655) (width 1.5) (layer B.Cu) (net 2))
 (segment (start 65.532 25.4) (end 65.532 28.147) (width 1.5) (layer B.Cu) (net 2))
 (via (at 50.927 30.21584) (size 0.8) (drill 0.45) (layers F.Cu B.Cu) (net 2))
 (segment (start 50.927 35.65) (end 50.927 30.21584) (width 0.2) (layer B.Cu) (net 2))
 (segment (start 50.509 36.068) (end 50.927 35.65) (width 0.2) (layer B.Cu) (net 2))
 (segment (start 49.36584 30.21584) (end 46.2518 27.1018) (width 0.35) (layer F.Cu) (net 2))
 (segment (start 50.927 30.21584) (end 49.36584 30.21584) (width 0.35) (layer F.Cu) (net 2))
 (via (at 48.768 23.283) (size 0.8) (drill 0.45) (layers F.Cu B.Cu) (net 2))
 (segment (start 46.2518 25.7992) (end 48.768 23.283) (width 1.5) (layer F.Cu) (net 2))
 (segment (start 46.2518 27.1018) (end 46.2518 25.7992) (width 1.5) (layer F.Cu) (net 2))
 (segment (start 43.28 24.13) (end 46.2518 27.1018) (width 1.5) (layer F.Cu) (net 2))
 (segment (start 42.23 24.13) (end 43.28 24.13) (width 1.5) (layer F.Cu) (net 2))
 (segment (start 65.659 34.036) (end 66.04 33.655) (width 1) (layer B.Cu) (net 12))
 (segment (start 62.354 34.036) (end 65.659 34.036) (width 1) (layer B.Cu) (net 12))
 (segment (start 62.354 34.036) (end 62.354 35.306) (width 0.2) (layer B.Cu) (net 12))
 (segment (start 31.115 25.89) (end 31.115 30.48) (width 1.5) (layer B.Cu) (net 15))
 (segment (start 30.335 26.67) (end 31.115 25.89) (width 1.5) (layer B.Cu) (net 15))
 (segment (start 19.304 26.67) (end 30.335 26.67) (width 1.5) (layer B.Cu) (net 15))
 (segment (start 19.304 31.67) (end 25.48 31.67) (width 1.5) (layer B.Cu) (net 14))
 (segment (start 25.48 31.67) (end 27.305 29.845) (width 1.5) (layer B.Cu) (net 14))
 (via (at 27.305 29.845) (size 1.5) (drill 0.7) (layers F.Cu B.Cu) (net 14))
 (segment (start 27.305 29.845) (end 34.925 29.845) (width 1.5) (layer F.Cu) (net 14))
 (via (at 37.465 27.305) (size 1.5) (drill 0.7) (layers F.Cu B.Cu) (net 14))
 (segment (start 34.925 29.845) (end 37.465 27.305) (width 1.5) (layer F.Cu) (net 14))
 (segment (start 37.465 25.89) (end 37.465 27.305) (width 1.5) (layer B.Cu) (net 14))
 (segment (start 37.465 27.305) (end 37.465 28.575) (width 1.5) (layer B.Cu) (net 14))
 (segment (start 37.465 28.575) (end 37.465 30.48) (width 1.5) (layer B.Cu) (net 14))
 (segment (start 19.614001 36.980001) (end 23.344999 36.980001) (width 1.5) (layer B.Cu) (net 13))
 (segment (start 19.304 36.67) (end 19.614001 36.980001) (width 1.5) (layer B.Cu) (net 13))
 (via (at 27.94 32.385) (size 1.5) (drill 0.7) (layers F.Cu B.Cu) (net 13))
 (segment (start 23.344999 36.980001) (end 27.94 32.385) (width 1.5) (layer B.Cu) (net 13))
 (segment (start 27.94 32.385) (end 28.575 31.75) (width 1.5) (layer F.Cu) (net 13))
 (via (at 43.18 30.48) (size 1.5) (drill 0.7) (layers F.Cu B.Cu) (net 13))
 (segment (start 41.91 31.75) (end 43.18 30.48) (width 1.5) (layer F.Cu) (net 13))
 (segment (start 28.575 31.75) (end 41.91 31.75) (width 1.5) (layer F.Cu) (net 13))
 (segment (start 43.18 30.48) (end 43.18 29.21) (width 1.5) (layer B.Cu) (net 13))
 (segment (start 43.18 25.89) (end 43.18 29.21) (width 1.5) (layer B.Cu) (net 13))
 (segment (start 56.12899 31.526176) (end 57.320166 30.335) (width 0.2) (layer B.Cu) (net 7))
 (segment (start 56.12899 36.239598) (end 56.12899 31.526176) (width 0.2) (layer B.Cu) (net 7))
 (segment (start 55.650588 36.718) (end 56.12899 36.239598) (width 0.2) (layer B.Cu) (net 7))
 (segment (start 54.084 36.718) (end 55.650588 36.718) (width 0.2) (layer B.Cu) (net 7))
 (via (at 55.626 37.592) (size 0.8) (drill 0.3) (layers F.Cu B.Cu) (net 7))
 (segment (start 55.626 36.742588) (end 55.650588 36.718) (width 0.2) (layer B.Cu) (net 7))
 (segment (start 55.626 37.592) (end 55.626 36.742588) (width 0.2) (layer B.Cu) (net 7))
 (segment (start 55.626 37.592) (end 55.4228 37.3888) (width 0.2) (layer F.Cu) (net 7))
 (segment (start 40.5638 37.3888) (end 37.465 34.29) (width 0.2) (layer F.Cu) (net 7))
 (segment (start 55.4228 37.3888) (end 40.5638 37.3888) (width 0.2) (layer F.Cu) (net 7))
 (segment (start 60.19822 30.335) (end 60.5991 30.335) (width 0.35) (layer B.Cu) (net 7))
 (segment (start 57.320166 30.335) (end 60.19822 30.335) (width 0.2) (layer B.Cu) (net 7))
 (segment (start 60.19822 30.335) (end 60.325 30.335) (width 0.2) (layer B.Cu) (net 7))
 (segment (start 61.232 29.7021) (end 61.232 25.4) (width 0.35) (layer B.Cu) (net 7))
 (segment (start 60.5991 30.335) (end 61.232 29.7021) (width 0.35) (layer B.Cu) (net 7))
 (segment (start 54.084 40.1902) (end 59.182 45.2882) (width 0.8) (layer B.Cu) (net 3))
 (segment (start 59.182 38.956) (end 59.182 45.2882) (width 1.5) (layer F.Cu) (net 3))
 (segment (start 42.865 34.29) (end 44.5668 35.9918) (width 1.5) (layer F.Cu) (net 3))
 (segment (start 56.2178 35.9918) (end 59.182 38.956) (width 1.5) (layer F.Cu) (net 3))
 (segment (start 44.5668 35.9918) (end 56.2178 35.9918) (width 1.5) (layer F.Cu) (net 3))
 (segment (start 27.94 48.006) (end 38.862 48.006) (width 1.5) (layer F.Cu) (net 3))
 (segment (start 27.6225 45.212) (end 27.6225 47.6885) (width 1.5) (layer F.Cu) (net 3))
 (segment (start 51.054 45.466) (end 53.086 47.498) (width 1.5) (layer F.Cu) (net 3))
 (segment (start 27.6225 47.6885) (end 27.94 48.006) (width 1.5) (layer F.Cu) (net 3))
 (segment (start 41.402 45.466) (end 51.054 45.466) (width 1.5) (layer F.Cu) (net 3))
 (segment (start 53.086 47.498) (end 59.182 47.498) (width 1.5) (layer F.Cu) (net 3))
 (segment (start 59.182 45.2882) (end 59.182 47.498) (width 1.5) (layer F.Cu) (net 3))
 (segment (start 38.862 48.006) (end 41.402 45.466) (width 1.5) (layer F.Cu) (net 3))
 (segment (start 45.565 31.59) (end 42.865 34.29) (width 1.5) (layer F.Cu) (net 3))
 (segment (start 51.816 31.59) (end 45.565 31.59) (width 1.5) (layer F.Cu) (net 3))
 (segment (start 58.7518 27.1018) (end 56.3042 27.1018) (width 1.5) (layer F.Cu) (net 3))
 (segment (start 54.084 38.018) (end 54.084 40.1902) (width 0.35) (layer B.Cu) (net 3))
 (segment (start 56.3042 27.1018) (end 51.816 31.59) (width 1.5) (layer F.Cu) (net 3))
 (segment (start 32.7025 45.212) (end 50.8 45.212) (width 0.8) (layer B.Cu) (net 6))
 (segment (start 50.8 45.212) (end 50.8 40.011298) (width 0.8) (layer B.Cu) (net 6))
 (segment (start 50.8 40.011298) (end 51.247649 39.563649) (width 0.8) (layer B.Cu) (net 6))
 (segment (start 51.354551 39.563649) (end 51.247649 39.563649) (width 0.35) (layer B.Cu) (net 6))
 (segment (start 52.809001 38.109199) (end 51.354551 39.563649) (width 0.35) (layer B.Cu) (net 6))
 (segment (start 52.809001 37.896231) (end 52.809001 38.109199) (width 0.35) (layer B.Cu) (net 6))
 (segment (start 53.337232 37.368) (end 52.809001 37.896231) (width 0.35) (layer B.Cu) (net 6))
 (segment (start 54.084 37.368) (end 53.337232 37.368) (width 0.35) (layer B.Cu) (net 6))
 (segment (start 54.084 34.768) (end 54.084 34.2826) (width 0.2) (layer B.Cu) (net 10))
 (via (at 54.084 34.2826) (size 0.8) (drill 0.45) (layers F.Cu B.Cu) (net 10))
 (segment (start 54.084 34.2826) (end 54.537401 34.736001) (width 0.2) (layer F.Cu) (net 10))
 (via (at 58.104 35.604905) (size 0.8) (drill 0.45) (layers F.Cu B.Cu) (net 10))
 (segment (start 57.235096 34.736001) (end 58.104 35.604905) (width 0.2) (layer F.Cu) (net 10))
 (segment (start 54.537401 34.736001) (end 57.235096 34.736001) (width 0.2) (layer F.Cu) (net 10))
 (segment (start 33.647684 37.368) (end 29.613684 41.402) (width 0.8) (layer B.Cu) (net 5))
 (segment (start 29.613684 41.402) (end 27.178 41.402) (width 0.8) (layer B.Cu) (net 5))
 (segment (start 27.178 41.402) (end 24.638 43.942) (width 0.8) (layer B.Cu) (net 5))
 (segment (start 24.638 44.046316) (end 24.384 44.300316) (width 0.8) (layer B.Cu) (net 5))
 (segment (start 24.638 43.942) (end 24.638 44.046316) (width 0.8) (layer B.Cu) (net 5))
 (segment (start 24.384 48.006) (end 26.67 50.292) (width 0.8) (layer B.Cu) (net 5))
 (segment (start 24.384 44.300316) (end 24.384 48.006) (width 0.8) (layer B.Cu) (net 5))
 (segment (start 26.67 50.292) (end 61.722 50.292) (width 0.8) (layer B.Cu) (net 5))
 (segment (start 61.722 45.2882) (end 61.722 46.5836) (width 0.8) (layer B.Cu) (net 5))
 (segment (start 61.722 46.5836) (end 61.722 45.1485) (width 0.8) (layer B.Cu) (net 5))
 (segment (start 61.722 50.292) (end 61.722 46.5836) (width 0.8) (layer B.Cu) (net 5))
 (segment (start 45.3436 37.368) (end 49.784 37.368) (width 0.35) (layer B.Cu) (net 5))
 (segment (start 45.3436 37.368) (end 33.647684 37.368) (width 0.8) (layer B.Cu) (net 5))
 (via (at 57.404 34.036) (size 0.8) (drill 0.3) (layers F.Cu B.Cu) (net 4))
 (via (at 57.2516 40.0812) (size 0.8) (drill 0.3) (layers F.Cu B.Cu) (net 4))
 (via (at 60.8838 40.0812) (size 0.8) (drill 0.3) (layers F.Cu B.Cu) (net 4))
 (via (at 51.133999 38.637199) (size 0.8) (drill 0.3) (layers F.Cu B.Cu) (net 4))
 (segment (start 57.2516 40.0812) (end 60.8838 40.0812) (width 0.2) (layer B.Cu) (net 4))
 (segment (start 56.8706 34.036) (end 57.404 34.036) (width 0.2) (layer B.Cu) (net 4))
 (segment (start 55.807599 38.637199) (end 57.2516 40.0812) (width 0.2) (layer F.Cu) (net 4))
 (segment (start 51.133999 37.342999) (end 51.133999 38.637199) (width 0.2) (layer B.Cu) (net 4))
 (segment (start 49.784 36.718) (end 50.509 36.718) (width 0.2) (layer B.Cu) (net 4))
 (segment (start 50.509 36.718) (end 51.133999 37.342999) (width 0.2) (layer B.Cu) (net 4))
 (segment (start 51.133999 38.637199) (end 55.807599 38.637199) (width 0.2) (layer F.Cu) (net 4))
 (segment (start 57.404 34.036) (end 59.6392 34.036) (width 0.2) (layer F.Cu) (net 4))
 (segment (start 60.8838 35.2806) (end 60.8838 38.1762) (width 0.2) (layer F.Cu) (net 4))
 (segment (start 59.6392 34.036) (end 60.8838 35.2806) (width 0.2) (layer F.Cu) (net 4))
 (segment (start 60.8838 40.0812) (end 60.8838 38.1762) (width 0.2) (layer F.Cu) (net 4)))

